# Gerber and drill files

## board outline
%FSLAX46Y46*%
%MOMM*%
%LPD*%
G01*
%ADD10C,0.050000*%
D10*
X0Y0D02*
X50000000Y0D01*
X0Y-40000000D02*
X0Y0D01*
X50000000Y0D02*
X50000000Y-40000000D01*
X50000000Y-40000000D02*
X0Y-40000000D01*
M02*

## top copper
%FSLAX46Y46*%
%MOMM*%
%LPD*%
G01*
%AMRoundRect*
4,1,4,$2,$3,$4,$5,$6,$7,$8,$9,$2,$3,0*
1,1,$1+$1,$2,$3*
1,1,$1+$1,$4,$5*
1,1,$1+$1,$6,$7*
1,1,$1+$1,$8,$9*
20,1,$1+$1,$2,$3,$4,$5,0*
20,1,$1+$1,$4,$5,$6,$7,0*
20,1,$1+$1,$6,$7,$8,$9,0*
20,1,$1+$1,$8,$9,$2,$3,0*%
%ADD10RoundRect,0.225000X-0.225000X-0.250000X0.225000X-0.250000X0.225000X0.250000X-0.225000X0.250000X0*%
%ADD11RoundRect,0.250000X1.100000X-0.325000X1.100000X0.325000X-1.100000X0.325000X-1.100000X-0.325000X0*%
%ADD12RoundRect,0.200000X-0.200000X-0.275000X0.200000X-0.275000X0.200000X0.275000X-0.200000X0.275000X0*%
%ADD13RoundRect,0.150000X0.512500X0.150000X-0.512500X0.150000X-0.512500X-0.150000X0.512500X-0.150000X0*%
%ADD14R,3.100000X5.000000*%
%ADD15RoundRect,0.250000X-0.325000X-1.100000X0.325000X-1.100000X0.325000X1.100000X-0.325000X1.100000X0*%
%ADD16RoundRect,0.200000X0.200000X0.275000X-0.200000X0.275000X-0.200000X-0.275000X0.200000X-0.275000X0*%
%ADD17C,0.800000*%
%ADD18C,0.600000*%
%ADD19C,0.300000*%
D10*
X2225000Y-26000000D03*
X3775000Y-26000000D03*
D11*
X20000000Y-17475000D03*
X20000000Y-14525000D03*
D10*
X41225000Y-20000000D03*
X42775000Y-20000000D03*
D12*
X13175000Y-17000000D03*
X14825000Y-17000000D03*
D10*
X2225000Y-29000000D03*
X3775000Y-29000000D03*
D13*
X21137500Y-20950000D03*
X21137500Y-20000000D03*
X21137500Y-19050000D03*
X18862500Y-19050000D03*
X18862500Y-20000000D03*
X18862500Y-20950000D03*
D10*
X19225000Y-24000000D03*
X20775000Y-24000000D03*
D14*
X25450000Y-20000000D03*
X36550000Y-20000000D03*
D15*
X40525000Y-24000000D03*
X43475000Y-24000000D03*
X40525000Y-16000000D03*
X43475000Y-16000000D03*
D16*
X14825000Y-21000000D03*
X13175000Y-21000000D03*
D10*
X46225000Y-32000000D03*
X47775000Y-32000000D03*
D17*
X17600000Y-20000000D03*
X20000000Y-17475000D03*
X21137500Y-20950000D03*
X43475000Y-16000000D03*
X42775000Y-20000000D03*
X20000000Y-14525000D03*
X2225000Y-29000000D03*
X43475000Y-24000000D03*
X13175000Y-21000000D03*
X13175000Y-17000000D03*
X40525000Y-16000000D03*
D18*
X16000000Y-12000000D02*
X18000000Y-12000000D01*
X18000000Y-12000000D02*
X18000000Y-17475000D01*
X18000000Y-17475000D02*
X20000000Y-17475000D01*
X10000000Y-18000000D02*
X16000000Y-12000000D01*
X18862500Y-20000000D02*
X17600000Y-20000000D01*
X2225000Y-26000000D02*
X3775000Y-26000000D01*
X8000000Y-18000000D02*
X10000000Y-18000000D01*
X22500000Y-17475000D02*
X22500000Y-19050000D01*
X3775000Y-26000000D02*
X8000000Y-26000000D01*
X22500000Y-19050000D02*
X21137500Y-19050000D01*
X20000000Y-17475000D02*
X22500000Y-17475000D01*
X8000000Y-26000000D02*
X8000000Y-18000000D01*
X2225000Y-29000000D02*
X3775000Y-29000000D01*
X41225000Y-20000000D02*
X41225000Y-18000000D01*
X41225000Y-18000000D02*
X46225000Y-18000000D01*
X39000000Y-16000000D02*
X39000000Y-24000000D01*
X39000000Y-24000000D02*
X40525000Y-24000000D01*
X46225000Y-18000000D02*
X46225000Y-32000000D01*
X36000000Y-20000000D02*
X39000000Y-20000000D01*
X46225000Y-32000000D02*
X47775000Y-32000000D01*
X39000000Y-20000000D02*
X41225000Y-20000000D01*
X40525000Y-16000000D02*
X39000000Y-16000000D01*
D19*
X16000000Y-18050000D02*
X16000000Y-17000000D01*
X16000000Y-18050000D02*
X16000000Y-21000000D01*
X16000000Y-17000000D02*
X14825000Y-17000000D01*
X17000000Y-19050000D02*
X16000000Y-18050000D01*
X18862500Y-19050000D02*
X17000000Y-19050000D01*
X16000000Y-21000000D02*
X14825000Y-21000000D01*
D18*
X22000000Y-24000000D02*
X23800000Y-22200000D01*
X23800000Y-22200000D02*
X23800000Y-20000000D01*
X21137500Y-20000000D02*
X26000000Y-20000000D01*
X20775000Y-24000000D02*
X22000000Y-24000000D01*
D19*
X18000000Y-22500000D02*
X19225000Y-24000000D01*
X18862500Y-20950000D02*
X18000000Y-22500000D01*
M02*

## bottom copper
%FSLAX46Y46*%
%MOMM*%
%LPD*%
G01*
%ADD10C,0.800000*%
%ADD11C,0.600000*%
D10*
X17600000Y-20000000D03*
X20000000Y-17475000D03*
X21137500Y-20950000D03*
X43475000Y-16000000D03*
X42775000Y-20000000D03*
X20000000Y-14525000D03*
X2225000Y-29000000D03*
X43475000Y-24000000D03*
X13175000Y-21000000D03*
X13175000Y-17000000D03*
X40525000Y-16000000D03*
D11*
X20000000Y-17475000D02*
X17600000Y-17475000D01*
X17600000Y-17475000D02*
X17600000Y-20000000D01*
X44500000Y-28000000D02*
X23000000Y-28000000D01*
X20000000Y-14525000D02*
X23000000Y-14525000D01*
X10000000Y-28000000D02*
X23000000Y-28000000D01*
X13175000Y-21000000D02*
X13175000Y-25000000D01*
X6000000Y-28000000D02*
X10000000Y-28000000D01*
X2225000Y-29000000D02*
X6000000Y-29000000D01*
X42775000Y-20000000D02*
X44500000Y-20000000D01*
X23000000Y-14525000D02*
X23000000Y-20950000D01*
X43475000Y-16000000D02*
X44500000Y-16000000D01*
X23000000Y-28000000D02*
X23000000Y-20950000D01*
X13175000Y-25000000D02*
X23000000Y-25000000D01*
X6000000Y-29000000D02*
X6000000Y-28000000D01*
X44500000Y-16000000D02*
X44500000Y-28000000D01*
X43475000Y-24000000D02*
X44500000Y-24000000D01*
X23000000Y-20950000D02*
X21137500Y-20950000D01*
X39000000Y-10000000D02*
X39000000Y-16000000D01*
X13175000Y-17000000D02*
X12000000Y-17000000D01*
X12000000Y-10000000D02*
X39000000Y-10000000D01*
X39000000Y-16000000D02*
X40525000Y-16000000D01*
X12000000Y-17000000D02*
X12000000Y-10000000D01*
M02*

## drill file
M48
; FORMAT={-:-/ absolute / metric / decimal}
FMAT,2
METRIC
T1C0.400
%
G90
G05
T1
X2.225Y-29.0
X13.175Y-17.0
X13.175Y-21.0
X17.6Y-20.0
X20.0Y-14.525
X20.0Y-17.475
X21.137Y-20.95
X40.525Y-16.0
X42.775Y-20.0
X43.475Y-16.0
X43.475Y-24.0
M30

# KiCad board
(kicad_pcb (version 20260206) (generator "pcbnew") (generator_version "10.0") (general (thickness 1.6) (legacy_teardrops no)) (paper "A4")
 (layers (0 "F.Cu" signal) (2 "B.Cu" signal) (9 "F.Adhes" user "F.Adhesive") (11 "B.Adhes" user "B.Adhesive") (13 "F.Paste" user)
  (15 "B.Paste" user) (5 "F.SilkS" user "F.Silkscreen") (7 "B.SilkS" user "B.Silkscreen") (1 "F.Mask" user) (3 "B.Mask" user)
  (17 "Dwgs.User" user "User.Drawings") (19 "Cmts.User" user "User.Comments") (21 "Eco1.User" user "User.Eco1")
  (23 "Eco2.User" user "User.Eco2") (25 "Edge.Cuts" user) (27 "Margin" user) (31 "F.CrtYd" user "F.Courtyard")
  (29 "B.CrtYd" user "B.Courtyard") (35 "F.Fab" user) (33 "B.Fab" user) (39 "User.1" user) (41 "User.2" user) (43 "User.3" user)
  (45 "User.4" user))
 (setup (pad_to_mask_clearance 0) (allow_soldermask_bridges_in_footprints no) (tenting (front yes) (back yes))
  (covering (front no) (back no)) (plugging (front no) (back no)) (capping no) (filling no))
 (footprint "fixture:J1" (layer "F.Cu") (at 3 26)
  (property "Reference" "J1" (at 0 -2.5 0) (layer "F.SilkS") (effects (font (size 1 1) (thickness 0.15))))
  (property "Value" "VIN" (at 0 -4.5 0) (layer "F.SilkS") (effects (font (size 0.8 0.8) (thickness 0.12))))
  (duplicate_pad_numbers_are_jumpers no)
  (pad "1" smd roundrect (at -0.775 0) (size 0.9 0.95) (layers "F.Cu" "F.Mask" "F.Paste") (roundrect_rratio 0.25) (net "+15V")
   (thermal_bridge_angle 45))
  (pad "2" smd roundrect (at 0.775 0) (size 0.9 0.95) (layers "F.Cu" "F.Mask" "F.Paste") (roundrect_rratio 0.25) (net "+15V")
   (thermal_bridge_angle 45)))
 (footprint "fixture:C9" (layer "F.Cu") (at 20 16 90)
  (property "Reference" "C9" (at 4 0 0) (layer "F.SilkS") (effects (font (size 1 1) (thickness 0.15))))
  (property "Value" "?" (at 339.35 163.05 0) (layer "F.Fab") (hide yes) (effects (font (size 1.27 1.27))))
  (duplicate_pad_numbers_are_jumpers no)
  (pad "1" smd roundrect (at -1.475 0 90) (size 1.15 2.7) (layers "F.Cu" "F.Mask" "F.Paste") (roundrect_rratio 0.217391) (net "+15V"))
  (pad "2" smd roundrect (at 1.475 0 90) (size 1.15 2.7) (layers "F.Cu" "F.Mask" "F.Paste") (roundrect_rratio 0.217391) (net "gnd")))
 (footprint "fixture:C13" (layer "F.Cu") (at 42 20)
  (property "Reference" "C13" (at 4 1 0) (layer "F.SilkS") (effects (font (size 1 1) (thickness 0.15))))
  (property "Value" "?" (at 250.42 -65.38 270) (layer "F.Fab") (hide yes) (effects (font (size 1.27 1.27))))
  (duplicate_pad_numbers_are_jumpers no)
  (pad "1" smd roundrect (at -0.775 0) (size 0.9 0.95) (layers "F.Cu" "F.Mask" "F.Paste") (roundrect_rratio 0.25) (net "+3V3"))
  (pad "2" smd roundrect (at 0.775 0) (size 0.9 0.95) (layers "F.Cu" "F.Mask" "F.Paste") (roundrect_rratio 0.25) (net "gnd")))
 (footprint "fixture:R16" (layer "F.Cu") (at 14 17)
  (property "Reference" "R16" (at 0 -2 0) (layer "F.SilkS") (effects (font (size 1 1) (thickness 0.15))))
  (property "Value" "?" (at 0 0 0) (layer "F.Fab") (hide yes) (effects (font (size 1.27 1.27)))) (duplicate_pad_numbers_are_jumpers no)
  (pad "1" smd roundrect (at -0.825 0) (size 0.8 0.95) (layers "F.Cu" "F.Mask" "F.Paste") (roundrect_rratio 0.25) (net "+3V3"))
  (pad "2" smd roundrect (at 0.825 0) (size 0.8 0.95) (layers "F.Cu" "F.Mask" "F.Paste") (roundrect_rratio 0.25) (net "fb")))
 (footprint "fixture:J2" (layer "F.Cu") (at 3 29)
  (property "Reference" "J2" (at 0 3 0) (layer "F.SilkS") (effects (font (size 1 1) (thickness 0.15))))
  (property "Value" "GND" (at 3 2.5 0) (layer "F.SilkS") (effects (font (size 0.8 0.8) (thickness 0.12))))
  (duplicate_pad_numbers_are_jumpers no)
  (pad "1" smd roundrect (at -0.775 0) (size 0.9 0.95) (layers "F.Cu" "F.Mask" "F.Paste") (roundrect_rratio 0.25) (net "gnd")
   (thermal_bridge_angle 45))
  (pad "2" smd roundrect (at 0.775 0) (size 0.9 0.95) (layers "F.Cu" "F.Mask" "F.Paste") (roundrect_rratio 0.25) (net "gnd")
   (thermal_bridge_angle 45)))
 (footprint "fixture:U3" (layer "F.Cu") (at 20 20 180)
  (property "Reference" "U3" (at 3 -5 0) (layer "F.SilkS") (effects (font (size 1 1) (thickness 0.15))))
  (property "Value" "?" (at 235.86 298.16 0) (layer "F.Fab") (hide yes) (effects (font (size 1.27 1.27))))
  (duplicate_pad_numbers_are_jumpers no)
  (pad "1" smd roundrect (at -1.1375 -0.95 180) (size 1.325 0.6) (layers "F.Cu" "F.Mask" "F.Paste") (roundrect_rratio 0.25) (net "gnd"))
  (pad "2" smd roundrect (at -1.1375 0 180) (size 1.325 0.6) (layers "F.Cu" "F.Mask" "F.Paste") (roundrect_rratio 0.25) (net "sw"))
  (pad "3" smd roundrect (at -1.1375 0.95 180) (size 1.325 0.6) (layers "F.Cu" "F.Mask" "F.Paste") (roundrect_rratio 0.25) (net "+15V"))
  (pad "4" smd roundrect (at 1.1375 0.95 180) (size 1.325 0.6) (layers "F.Cu" "F.Mask" "F.Paste") (roundrect_rratio 0.25) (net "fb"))
  (pad "5" smd roundrect (at 1.1375 0 180) (size 1.325 0.6) (layers "F.Cu" "F.Mask" "F.Paste") (roundrect_rratio 0.25) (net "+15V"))
  (pad "6" smd roundrect (at 1.1375 -0.95 180) (size 1.325 0.6) (layers "F.Cu" "F.Mask" "F.Paste") (roundrect_rratio 0.25) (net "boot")))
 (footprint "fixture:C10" (layer "F.Cu") (at 20 24)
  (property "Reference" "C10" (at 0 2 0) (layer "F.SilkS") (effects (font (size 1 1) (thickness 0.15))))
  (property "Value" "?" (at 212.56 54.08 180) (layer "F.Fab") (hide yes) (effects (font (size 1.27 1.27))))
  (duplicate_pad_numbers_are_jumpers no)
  (pad "1" smd roundrect (at -0.775 0) (size 0.9 0.95) (layers "F.Cu" "F.Mask" "F.Paste") (roundrect_rratio 0.25) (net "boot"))
  (pad "2" smd roundrect (at 0.775 0) (size 0.9 0.95) (layers "F.Cu" "F.Mask" "F.Paste") (roundrect_rratio 0.25) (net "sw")))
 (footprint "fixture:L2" (layer "F.Cu") (at 31 20)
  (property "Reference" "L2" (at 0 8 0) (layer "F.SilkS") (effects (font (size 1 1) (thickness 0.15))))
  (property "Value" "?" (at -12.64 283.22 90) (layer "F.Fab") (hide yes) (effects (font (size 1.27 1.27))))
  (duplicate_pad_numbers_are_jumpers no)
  (pad "1" smd rect (at -5.55 0) (size 3.1 5) (layers "F.Cu" "F.Mask" "F.Paste") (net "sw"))
  (pad "2" smd rect (at 5.55 0) (size 3.1 5) (layers "F.Cu" "F.Mask" "F.Paste") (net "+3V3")))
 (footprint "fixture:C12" (layer "F.Cu") (at 42 24)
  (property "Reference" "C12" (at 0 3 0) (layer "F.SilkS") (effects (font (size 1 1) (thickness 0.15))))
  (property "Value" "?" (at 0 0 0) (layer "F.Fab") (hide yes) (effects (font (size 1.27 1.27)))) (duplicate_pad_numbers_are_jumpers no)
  (pad "1" smd roundrect (at -1.475 0) (size 1.15 2.7) (layers "F.Cu" "F.Mask" "F.Paste") (roundrect_rratio 0.217391) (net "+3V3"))
  (pad "2" smd roundrect (at 1.475 0) (size 1.15 2.7) (layers "F.Cu" "F.Mask" "F.Paste") (roundrect_rratio 0.217391) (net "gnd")))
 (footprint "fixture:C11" (layer "F.Cu") (at 42 16)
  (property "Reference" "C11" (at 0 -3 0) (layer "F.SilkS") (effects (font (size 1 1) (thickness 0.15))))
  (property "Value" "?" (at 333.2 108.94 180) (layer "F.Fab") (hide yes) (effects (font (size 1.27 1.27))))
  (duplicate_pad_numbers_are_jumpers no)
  (pad "1" smd roundrect (at -1.475 0) (size 1.15 2.7) (layers "F.Cu" "F.Mask" "F.Paste") (roundrect_rratio 0.217391) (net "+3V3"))
  (pad "2" smd roundrect (at 1.475 0) (size 1.15 2.7) (layers "F.Cu" "F.Mask" "F.Paste") (roundrect_rratio 0.217391) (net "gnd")))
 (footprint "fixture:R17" (layer "F.Cu") (at 14 21 180)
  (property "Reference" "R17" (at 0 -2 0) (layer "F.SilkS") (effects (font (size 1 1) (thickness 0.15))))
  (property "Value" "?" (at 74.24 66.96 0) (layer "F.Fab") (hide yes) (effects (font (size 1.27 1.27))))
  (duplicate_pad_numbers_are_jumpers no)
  (pad "1" smd roundrect (at -0.825 0 180) (size 0.8 0.95) (layers "F.Cu" "F.Mask" "F.Paste") (roundrect_rratio 0.25) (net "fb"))
  (pad "2" smd roundrect (at 0.825 0 180) (size 0.8 0.95) (layers "F.Cu" "F.Mask" "F.Paste") (roundrect_rratio 0.25) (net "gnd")))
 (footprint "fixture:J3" (layer "F.Cu") (at 47 32)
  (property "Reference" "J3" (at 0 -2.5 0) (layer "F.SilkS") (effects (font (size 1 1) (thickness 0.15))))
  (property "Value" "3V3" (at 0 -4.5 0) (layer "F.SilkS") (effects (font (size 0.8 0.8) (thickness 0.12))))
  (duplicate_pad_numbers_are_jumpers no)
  (pad "1" smd roundrect (at -0.775 0) (size 0.9 0.95) (layers "F.Cu" "F.Mask" "F.Paste") (roundrect_rratio 0.25) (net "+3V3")
   (thermal_bridge_angle 45))
  (pad "2" smd roundrect (at 0.775 0) (size 0.9 0.95) (layers "F.Cu" "F.Mask" "F.Paste") (roundrect_rratio 0.25) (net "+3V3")
   (thermal_bridge_angle 45)))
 (gr_line (start 0 0) (end 50 0) (stroke (width 0.05) (type default)) (layer "Edge.Cuts"))
 (gr_line (start 0 40) (end 0 0) (stroke (width 0.05) (type default)) (layer "Edge.Cuts"))
 (gr_line (start 50 0) (end 50 40) (stroke (width 0.05) (type default)) (layer "Edge.Cuts"))
 (gr_line (start 50 40) (end 0 40) (stroke (width 0.05) (type default)) (layer "Edge.Cuts"))
 (segment (start 16 12) (end 18 12) (width 0.6) (layer "F.Cu") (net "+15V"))
 (segment (start 18 12) (end 18 17.475) (width 0.6) (layer "F.Cu") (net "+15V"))
 (segment (start 18 17.475) (end 20 17.475) (width 0.6) (layer "F.Cu") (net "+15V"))
 (segment (start 10 18) (end 16 12) (width 0.6) (layer "F.Cu") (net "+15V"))
 (segment (start 18.8625 20) (end 17.6 20) (width 0.6) (layer "F.Cu") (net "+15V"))
 (segment (start 2.225 26) (end 3.775 26) (width 0.6) (layer "F.Cu") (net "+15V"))
 (segment (start 8 18) (end 10 18) (width 0.6) (layer "F.Cu") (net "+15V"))
 (segment (start 22.5 17.475) (end 22.5 19.05) (width 0.6) (layer "F.Cu") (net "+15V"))
 (segment (start 3.775 26) (end 8 26) (width 0.6) (layer "F.Cu") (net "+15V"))
 (segment (start 22.5 19.05) (end 21.1375 19.05) (width 0.6) (layer "F.Cu") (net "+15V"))
 (segment (start 20 17.475) (end 22.5 17.475) (width 0.6) (layer "F.Cu") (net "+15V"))
 (segment (start 8 26) (end 8 18) (width 0.6) (layer "F.Cu") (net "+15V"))
 (via (at 17.6 20) (size 0.8) (drill 0.4) (layers "F.Cu" "B.Cu") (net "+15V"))
 (via (at 20 17.475) (size 0.8) (drill 0.4) (layers "F.Cu" "B.Cu") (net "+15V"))
 (segment (start 20 17.475) (end 17.6 17.475) (width 0.6) (layer "B.Cu") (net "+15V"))
 (segment (start 17.6 17.475) (end 17.6 20) (width 0.6) (layer "B.Cu") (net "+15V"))
 (segment (start 2.225 29) (end 3.775 29) (width 0.6) (layer "F.Cu") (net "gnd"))
 (via (at 21.1375 20.95) (size 0.8) (drill 0.4) (layers "F.Cu" "B.Cu") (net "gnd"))
 (via (at 43.475 16) (size 0.8) (drill 0.4) (layers "F.Cu" "B.Cu") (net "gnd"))
 (via (at 42.775 20) (size 0.8) (drill 0.4) (layers "F.Cu" "B.Cu") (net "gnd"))
 (via (at 20 14.525) (size 0.8) (drill 0.4) (layers "F.Cu" "B.Cu") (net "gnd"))
 (via (at 2.225 29) (size 0.8) (drill 0.4) (layers "F.Cu" "B.Cu") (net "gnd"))
 (via (at 43.475 24) (size 0.8) (drill 0.4) (layers "F.Cu" "B.Cu") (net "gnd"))
 (via (at 13.175 21) (size 0.8) (drill 0.4) (layers "F.Cu" "B.Cu") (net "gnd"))
 (segment (start 44.5 28) (end 23 28) (width 0.6) (layer "B.Cu") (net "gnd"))
 (segment (start 20 14.525) (end 23 14.525) (width 0.6) (layer "B.Cu") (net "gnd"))
 (segment (start 10 28) (end 23 28) (width 0.6) (layer "B.Cu") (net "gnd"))
 (segment (start 13.175 21) (end 13.175 25) (width 0.6) (layer "B.Cu") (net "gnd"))
 (segment (start 6 28) (end 10 28) (width 0.6) (layer "B.Cu") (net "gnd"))
 (segment (start 2.225 29) (end 6 29) (width 0.6) (layer "B.Cu") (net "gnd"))
 (segment (start 42.775 20) (end 44.5 20) (width 0.6) (layer "B.Cu") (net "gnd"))
 (segment (start 23 14.525) (end 23 20.95) (width 0.6) (layer "B.Cu") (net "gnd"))
 (segment (start 43.475 16) (end 44.5 16) (width 0.6) (layer "B.Cu") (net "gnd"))
 (segment (start 23 28) (end 23 20.95) (width 0.6) (layer "B.Cu") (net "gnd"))
 (segment (start 13.175 25) (end 23 25) (width 0.6) (layer "B.Cu") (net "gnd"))
 (segment (start 6 29) (end 6 28) (width 0.6) (layer "B.Cu") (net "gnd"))
 (segment (start 44.5 16) (end 44.5 28) (width 0.6) (layer "B.Cu") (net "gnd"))
 (segment (start 43.475 24) (end 44.5 24) (width 0.6) (layer "B.Cu") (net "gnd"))
 (segment (start 23 20.95) (end 21.1375 20.95) (width 0.6) (layer "B.Cu") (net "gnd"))
 (segment (start 41.225 20) (end 41.225 18) (width 0.6) (layer "F.Cu") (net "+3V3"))
 (segment (start 41.225 18) (end 46.225 18) (width 0.6) (layer "F.Cu") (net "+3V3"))
 (segment (start 39 16) (end 39 24) (width 0.6) (layer "F.Cu") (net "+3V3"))
 (segment (start 39 24) (end 40.525 24) (width 0.6) (layer "F.Cu") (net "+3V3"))
 (segment (start 46.225 18) (end 46.225 32) (width 0.6) (layer "F.Cu") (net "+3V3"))
 (segment (start 36 20) (end 39 20) (width 0.6) (layer "F.Cu") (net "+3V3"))
 (segment (start 46.225 32) (end 47.775 32) (width 0.6) (layer "F.Cu") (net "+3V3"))
 (segment (start 39 20) (end 41.225 20) (width 0.6) (layer "F.Cu") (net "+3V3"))
 (segment (start 40.525 16) (end 39 16) (width 0.6) (layer "F.Cu") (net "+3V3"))
 (via (at 13.175 17) (size 0.8) (drill 0.4) (layers "F.Cu" "B.Cu") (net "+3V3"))
 (via (at 40.525 16) (size 0.8) (drill 0.4) (layers "F.Cu" "B.Cu") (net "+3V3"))
 (segment (start 39 10) (end 39 16) (width 0.6) (layer "B.Cu") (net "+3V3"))
 (segment (start 13.175 17) (end 12 17) (width 0.6) (layer "B.Cu") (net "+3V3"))
 (segment (start 12 10) (end 39 10) (width 0.6) (layer "B.Cu") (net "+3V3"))
 (segment (start 39 16) (end 40.525 16) (width 0.6) (layer "B.Cu") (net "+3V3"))
 (segment (start 12 17) (end 12 10) (width 0.6) (layer "B.Cu") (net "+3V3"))
 (segment (start 16 18.05) (end 16 17) (width 0.3) (layer "F.Cu") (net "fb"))
 (segment (start 16 18.05) (end 16 21) (width 0.3) (layer "F.Cu") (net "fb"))
 (segment (start 16 17) (end 14.825 17) (width 0.3) (layer "F.Cu") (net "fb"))
 (segment (start 17 19.05) (end 16 18.05) (width 0.3) (layer "F.Cu") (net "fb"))
 (segment (start 18.8625 19.05) (end 17 19.05) (width 0.3) (layer "F.Cu") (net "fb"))
 (segment (start 16 21) (end 14.825 21) (width 0.3) (layer "F.Cu") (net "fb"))
 (segment (start 22 24) (end 23.8 22.2) (width 0.6) (layer "F.Cu") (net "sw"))
 (segment (start 23.8 22.2) (end 23.8 20) (width 0.6) (layer "F.Cu") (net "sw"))
 (segment (start 21.1375 20) (end 26 20) (width 0.6) (layer "F.Cu") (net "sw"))
 (segment (start 20.775 24) (end 22 24) (width 0.6) (layer "F.Cu") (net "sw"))
 (segment (start 18 22.5) (end 19.225 24) (width 0.3) (layer "F.Cu") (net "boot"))
 (segment (start 18.8625 20.95) (end 18 22.5) (width 0.3) (layer "F.Cu") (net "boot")))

